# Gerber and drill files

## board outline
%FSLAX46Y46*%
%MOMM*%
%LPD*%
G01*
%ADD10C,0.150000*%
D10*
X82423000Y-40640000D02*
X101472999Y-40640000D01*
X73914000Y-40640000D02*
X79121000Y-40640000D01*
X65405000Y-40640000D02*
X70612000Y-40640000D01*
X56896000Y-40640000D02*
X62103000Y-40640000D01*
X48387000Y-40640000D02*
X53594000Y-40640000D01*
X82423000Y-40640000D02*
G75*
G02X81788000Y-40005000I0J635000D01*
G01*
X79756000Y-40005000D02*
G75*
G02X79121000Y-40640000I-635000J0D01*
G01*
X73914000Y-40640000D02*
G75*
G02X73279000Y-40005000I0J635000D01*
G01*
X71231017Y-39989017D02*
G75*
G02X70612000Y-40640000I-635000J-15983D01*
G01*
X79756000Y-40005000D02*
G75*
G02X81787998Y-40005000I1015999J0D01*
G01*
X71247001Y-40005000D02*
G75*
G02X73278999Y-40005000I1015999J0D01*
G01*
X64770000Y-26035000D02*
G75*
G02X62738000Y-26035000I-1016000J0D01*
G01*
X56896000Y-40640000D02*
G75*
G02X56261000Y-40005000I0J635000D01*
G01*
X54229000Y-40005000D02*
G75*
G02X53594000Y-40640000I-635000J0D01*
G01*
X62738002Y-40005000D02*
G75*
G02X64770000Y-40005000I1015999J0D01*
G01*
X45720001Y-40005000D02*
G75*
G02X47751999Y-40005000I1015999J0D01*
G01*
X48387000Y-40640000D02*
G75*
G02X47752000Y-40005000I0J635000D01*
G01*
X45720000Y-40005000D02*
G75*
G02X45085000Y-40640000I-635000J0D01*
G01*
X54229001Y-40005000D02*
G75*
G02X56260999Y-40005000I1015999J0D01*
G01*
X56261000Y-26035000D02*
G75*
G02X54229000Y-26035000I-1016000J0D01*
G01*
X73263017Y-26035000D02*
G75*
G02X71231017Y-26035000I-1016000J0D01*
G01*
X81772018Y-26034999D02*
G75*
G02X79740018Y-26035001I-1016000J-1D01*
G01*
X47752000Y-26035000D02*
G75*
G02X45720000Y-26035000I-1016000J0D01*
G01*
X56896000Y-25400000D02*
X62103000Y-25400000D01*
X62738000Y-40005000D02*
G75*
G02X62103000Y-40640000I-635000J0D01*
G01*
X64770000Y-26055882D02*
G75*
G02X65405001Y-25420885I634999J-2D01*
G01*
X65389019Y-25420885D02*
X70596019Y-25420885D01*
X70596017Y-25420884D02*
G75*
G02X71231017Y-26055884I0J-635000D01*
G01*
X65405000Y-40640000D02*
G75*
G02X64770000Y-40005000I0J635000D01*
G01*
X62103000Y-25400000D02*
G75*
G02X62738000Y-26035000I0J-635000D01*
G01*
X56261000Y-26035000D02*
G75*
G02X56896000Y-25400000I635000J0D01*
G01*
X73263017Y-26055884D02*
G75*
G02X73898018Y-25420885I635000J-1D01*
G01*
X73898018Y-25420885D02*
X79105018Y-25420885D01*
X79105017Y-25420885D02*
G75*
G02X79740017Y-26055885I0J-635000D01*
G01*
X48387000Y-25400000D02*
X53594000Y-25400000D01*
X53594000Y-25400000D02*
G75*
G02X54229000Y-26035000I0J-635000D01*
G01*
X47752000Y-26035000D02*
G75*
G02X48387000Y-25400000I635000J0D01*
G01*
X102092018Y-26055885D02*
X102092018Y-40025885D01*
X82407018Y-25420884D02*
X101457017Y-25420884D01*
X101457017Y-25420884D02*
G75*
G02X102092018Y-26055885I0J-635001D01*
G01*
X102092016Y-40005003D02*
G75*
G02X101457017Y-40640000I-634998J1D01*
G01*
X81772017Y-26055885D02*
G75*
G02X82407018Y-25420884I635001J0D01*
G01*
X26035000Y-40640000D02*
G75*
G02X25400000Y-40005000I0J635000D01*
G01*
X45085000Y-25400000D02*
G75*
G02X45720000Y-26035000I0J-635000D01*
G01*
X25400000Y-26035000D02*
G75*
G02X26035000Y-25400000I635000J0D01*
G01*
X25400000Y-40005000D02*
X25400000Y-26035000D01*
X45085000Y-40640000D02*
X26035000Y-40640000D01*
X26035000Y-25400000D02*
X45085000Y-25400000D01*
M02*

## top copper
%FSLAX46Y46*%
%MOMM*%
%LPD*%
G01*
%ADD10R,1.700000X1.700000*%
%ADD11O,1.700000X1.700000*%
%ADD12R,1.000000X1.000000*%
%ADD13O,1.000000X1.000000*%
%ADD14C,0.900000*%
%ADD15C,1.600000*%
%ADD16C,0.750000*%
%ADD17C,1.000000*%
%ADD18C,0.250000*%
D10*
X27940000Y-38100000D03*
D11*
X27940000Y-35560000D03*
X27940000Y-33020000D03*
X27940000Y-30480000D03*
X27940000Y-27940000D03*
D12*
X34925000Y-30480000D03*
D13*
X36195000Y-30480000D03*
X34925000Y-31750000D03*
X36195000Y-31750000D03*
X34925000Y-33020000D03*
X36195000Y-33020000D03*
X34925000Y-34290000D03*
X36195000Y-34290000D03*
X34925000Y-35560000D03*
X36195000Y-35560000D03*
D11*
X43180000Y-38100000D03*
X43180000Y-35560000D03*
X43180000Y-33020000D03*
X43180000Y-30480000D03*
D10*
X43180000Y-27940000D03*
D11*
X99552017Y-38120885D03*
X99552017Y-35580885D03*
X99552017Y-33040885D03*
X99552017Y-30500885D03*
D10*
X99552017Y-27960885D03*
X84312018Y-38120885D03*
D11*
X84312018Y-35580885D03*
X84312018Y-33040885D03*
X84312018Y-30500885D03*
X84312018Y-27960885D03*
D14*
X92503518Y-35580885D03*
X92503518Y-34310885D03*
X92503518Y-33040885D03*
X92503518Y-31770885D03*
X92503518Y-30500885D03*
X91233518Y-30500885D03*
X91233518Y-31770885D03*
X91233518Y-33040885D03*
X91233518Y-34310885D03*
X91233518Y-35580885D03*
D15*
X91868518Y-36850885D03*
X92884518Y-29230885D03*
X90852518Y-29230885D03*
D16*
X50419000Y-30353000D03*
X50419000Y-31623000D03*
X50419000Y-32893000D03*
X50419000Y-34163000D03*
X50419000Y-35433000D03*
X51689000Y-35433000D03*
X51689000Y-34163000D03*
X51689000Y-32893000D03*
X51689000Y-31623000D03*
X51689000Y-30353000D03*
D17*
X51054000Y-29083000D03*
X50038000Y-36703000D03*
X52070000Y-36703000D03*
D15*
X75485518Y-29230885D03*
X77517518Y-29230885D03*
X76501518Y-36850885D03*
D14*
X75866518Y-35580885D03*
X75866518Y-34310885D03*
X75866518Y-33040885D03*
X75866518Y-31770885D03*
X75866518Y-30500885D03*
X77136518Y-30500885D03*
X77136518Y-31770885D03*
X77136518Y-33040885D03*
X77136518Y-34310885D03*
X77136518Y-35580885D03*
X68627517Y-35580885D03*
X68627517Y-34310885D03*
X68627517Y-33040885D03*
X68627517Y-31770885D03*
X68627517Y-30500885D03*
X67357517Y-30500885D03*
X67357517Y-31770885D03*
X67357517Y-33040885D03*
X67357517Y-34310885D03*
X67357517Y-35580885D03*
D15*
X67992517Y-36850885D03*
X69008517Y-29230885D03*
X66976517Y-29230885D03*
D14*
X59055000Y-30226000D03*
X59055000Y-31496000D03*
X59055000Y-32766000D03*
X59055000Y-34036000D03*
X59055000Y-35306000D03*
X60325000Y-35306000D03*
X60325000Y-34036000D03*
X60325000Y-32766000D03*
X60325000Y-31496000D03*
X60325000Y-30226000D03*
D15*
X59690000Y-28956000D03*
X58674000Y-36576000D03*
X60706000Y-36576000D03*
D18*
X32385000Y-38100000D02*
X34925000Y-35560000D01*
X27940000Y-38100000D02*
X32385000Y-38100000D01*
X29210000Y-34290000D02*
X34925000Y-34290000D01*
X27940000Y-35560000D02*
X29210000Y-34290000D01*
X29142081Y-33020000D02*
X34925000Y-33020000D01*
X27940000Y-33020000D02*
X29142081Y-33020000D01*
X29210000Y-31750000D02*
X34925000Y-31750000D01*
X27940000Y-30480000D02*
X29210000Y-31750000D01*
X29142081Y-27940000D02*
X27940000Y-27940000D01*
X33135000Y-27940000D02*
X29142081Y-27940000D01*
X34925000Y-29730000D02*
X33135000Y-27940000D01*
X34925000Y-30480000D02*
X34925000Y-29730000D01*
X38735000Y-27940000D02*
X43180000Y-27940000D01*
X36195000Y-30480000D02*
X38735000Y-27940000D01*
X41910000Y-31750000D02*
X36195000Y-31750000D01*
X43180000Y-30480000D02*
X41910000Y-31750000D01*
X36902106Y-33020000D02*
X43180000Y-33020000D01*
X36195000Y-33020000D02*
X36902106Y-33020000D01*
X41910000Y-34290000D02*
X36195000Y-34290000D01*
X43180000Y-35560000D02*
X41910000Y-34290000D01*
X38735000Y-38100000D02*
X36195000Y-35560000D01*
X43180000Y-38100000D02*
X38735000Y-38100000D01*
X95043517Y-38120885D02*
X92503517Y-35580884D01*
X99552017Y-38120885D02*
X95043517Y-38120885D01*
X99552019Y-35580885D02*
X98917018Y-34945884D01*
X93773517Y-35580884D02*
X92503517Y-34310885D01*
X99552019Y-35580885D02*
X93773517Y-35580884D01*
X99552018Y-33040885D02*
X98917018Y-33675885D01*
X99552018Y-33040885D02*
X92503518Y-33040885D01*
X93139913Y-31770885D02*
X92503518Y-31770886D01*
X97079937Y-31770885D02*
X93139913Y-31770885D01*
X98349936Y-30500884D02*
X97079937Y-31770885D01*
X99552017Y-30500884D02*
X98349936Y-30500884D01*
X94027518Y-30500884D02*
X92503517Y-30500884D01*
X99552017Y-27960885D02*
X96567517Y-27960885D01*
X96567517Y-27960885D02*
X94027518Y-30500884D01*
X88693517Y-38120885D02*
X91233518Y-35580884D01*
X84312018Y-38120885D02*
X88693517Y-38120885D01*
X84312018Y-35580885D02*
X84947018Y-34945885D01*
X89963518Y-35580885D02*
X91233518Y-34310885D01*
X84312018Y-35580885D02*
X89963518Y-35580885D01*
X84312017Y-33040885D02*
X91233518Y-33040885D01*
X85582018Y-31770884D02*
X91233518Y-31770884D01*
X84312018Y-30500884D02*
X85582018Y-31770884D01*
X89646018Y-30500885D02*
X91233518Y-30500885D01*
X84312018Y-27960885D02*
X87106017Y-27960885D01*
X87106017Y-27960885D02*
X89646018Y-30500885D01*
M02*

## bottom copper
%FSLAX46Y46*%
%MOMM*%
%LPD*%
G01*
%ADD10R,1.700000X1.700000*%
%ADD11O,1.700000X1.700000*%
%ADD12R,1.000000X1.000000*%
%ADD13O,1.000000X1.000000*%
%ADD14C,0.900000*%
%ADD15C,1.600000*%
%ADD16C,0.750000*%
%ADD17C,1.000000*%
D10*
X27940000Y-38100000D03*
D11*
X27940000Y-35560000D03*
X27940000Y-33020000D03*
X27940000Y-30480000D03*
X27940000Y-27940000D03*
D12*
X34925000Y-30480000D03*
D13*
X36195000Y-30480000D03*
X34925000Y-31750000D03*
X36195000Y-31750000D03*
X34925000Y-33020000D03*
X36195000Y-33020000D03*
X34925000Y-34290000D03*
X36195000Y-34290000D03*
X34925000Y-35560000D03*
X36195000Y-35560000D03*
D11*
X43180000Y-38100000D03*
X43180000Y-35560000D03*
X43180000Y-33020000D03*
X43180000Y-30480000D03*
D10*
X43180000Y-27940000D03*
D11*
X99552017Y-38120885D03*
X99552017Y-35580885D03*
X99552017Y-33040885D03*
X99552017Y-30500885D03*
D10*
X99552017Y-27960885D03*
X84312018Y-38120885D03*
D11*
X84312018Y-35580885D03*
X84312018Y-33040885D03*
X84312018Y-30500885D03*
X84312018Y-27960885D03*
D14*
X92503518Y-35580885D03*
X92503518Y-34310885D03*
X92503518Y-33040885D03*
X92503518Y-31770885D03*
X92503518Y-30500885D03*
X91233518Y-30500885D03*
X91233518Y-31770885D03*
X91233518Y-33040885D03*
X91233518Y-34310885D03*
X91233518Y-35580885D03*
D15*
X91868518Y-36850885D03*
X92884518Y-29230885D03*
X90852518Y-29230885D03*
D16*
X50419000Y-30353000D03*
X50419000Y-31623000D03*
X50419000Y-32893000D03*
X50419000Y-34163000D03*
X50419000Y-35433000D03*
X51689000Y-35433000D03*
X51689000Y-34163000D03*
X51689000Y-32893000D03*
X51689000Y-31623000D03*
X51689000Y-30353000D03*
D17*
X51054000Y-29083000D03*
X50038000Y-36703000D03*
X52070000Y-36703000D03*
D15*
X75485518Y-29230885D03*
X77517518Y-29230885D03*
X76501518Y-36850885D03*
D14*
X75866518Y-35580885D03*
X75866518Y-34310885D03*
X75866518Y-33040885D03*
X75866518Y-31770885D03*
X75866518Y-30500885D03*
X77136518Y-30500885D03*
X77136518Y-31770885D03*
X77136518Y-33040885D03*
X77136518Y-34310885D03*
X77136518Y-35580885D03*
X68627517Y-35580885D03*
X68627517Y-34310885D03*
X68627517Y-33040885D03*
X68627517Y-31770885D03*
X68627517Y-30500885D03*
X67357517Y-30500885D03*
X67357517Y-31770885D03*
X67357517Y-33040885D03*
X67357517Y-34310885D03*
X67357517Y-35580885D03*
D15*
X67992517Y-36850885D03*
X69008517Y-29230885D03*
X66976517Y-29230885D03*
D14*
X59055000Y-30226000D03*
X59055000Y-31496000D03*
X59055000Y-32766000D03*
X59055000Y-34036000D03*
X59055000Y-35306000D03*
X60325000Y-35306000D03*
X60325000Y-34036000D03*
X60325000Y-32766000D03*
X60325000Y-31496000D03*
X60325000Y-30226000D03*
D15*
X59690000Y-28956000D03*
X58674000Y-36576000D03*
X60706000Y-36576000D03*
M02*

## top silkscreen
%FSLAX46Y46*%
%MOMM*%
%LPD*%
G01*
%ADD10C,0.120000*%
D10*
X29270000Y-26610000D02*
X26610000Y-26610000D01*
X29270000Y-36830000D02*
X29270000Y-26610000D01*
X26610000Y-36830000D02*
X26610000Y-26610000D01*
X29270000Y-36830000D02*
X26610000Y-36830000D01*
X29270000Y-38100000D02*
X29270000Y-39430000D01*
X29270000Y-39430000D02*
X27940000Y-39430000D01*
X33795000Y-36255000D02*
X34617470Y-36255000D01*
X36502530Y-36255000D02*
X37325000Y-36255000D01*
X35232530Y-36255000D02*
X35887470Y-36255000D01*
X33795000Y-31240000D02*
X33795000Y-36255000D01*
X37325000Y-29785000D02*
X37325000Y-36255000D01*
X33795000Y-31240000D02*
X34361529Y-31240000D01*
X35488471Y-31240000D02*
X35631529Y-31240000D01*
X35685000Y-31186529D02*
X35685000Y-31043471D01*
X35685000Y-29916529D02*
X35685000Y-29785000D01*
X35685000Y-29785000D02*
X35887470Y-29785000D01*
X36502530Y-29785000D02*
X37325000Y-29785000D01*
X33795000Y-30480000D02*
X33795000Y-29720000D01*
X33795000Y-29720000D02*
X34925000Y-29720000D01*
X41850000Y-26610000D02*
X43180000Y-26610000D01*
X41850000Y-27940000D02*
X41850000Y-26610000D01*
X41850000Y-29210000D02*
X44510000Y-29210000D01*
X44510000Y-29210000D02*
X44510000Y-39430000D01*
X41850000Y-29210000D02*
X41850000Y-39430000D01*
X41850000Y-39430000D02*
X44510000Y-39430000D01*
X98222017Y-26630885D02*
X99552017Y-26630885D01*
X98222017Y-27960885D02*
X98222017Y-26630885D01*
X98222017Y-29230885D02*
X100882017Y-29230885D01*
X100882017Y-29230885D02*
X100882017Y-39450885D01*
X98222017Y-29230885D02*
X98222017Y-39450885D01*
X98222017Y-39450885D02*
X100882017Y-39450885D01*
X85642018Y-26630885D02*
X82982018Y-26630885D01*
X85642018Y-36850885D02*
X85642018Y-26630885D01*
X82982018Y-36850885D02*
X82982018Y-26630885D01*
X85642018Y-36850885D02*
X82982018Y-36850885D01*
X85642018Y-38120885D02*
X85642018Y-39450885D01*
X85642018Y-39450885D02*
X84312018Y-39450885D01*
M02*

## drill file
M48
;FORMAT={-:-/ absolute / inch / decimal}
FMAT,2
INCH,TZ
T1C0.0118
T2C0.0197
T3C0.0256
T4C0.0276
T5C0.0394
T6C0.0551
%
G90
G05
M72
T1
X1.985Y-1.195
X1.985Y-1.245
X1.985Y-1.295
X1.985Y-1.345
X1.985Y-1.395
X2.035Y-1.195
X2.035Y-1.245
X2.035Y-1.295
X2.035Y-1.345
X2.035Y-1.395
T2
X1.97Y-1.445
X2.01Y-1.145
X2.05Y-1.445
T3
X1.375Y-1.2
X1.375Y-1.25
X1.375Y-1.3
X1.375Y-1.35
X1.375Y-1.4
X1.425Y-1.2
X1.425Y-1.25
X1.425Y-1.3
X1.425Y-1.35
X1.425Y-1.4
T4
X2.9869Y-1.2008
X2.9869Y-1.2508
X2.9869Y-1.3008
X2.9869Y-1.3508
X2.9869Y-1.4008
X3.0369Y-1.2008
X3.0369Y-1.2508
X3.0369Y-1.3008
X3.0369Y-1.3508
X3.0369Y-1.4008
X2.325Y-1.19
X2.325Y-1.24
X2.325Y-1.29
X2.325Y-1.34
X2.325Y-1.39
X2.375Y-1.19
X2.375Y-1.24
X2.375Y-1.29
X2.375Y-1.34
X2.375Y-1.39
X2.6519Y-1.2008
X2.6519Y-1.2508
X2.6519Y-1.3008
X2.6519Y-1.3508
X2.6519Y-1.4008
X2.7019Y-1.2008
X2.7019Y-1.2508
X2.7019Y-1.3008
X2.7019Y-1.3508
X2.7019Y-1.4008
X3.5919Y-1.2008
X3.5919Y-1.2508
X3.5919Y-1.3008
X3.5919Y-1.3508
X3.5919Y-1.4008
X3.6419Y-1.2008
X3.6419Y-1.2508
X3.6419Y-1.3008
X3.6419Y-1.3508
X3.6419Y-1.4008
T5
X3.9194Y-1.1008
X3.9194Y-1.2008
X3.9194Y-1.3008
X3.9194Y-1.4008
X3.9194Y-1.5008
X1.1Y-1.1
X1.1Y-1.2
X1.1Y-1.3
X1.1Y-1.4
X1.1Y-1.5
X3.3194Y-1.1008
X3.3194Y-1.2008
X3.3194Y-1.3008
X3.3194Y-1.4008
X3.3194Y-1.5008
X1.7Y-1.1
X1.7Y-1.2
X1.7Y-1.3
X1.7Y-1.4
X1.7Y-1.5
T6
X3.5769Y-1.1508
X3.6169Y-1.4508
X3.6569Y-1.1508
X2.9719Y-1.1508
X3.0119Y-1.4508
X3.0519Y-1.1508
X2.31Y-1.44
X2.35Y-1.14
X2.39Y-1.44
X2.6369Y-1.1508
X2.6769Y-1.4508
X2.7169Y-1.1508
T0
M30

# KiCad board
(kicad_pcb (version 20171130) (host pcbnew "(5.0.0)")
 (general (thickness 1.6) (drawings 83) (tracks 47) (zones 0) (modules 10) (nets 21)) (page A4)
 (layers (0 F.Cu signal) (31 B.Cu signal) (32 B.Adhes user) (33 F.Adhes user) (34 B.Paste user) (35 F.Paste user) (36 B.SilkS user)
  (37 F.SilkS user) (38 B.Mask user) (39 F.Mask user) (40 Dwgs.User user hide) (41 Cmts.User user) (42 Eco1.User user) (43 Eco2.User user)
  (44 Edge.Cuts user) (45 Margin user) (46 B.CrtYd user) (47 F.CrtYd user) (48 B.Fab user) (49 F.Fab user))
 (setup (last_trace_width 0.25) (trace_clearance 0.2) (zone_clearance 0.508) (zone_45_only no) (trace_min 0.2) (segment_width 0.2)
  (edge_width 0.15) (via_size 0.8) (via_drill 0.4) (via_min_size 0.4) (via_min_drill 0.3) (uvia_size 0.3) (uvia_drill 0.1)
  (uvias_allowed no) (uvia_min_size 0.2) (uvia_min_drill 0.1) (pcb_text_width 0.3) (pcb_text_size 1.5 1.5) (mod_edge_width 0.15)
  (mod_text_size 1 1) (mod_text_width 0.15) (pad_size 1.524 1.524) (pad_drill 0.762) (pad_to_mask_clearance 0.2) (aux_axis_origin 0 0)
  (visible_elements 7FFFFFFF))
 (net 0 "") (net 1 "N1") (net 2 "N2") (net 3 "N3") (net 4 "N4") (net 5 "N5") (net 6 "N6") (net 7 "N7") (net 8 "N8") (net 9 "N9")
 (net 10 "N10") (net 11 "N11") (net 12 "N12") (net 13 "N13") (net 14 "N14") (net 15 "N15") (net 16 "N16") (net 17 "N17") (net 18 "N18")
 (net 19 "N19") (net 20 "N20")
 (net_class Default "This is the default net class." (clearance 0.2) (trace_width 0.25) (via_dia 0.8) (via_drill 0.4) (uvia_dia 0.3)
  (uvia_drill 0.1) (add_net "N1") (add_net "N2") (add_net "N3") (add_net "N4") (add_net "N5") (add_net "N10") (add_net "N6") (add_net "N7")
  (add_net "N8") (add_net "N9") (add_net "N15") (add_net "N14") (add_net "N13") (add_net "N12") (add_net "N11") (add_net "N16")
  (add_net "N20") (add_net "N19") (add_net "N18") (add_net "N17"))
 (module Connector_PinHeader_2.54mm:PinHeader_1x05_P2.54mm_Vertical (layer F.Cu) (at 27.94 38.1 180)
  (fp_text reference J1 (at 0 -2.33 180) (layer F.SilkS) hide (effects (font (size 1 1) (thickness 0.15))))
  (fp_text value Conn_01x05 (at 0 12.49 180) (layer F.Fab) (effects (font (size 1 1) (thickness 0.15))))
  (fp_line (start -1.33 11.49) (end 1.33 11.49) (layer F.SilkS) (width 0.12))
  (fp_line (start -1.33 1.27) (end -1.33 11.49) (layer F.SilkS) (width 0.12))
  (fp_line (start 1.33 1.27) (end 1.33 11.49) (layer F.SilkS) (width 0.12))
  (fp_line (start -1.33 1.27) (end 1.33 1.27) (layer F.SilkS) (width 0.12))
  (fp_line (start -1.33 0) (end -1.33 -1.33) (layer F.SilkS) (width 0.12))
  (fp_line (start -1.33 -1.33) (end 0 -1.33) (layer F.SilkS) (width 0.12))
  (pad 1 thru_hole rect (at 0 0 180) (size 1.7 1.7) (drill 1) (layers *.Cu *.Mask) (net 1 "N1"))
  (pad 2 thru_hole oval (at 0 2.54 180) (size 1.7 1.7) (drill 1) (layers *.Cu *.Mask) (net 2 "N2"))
  (pad 3 thru_hole oval (at 0 5.08 180) (size 1.7 1.7) (drill 1) (layers *.Cu *.Mask) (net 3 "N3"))
  (pad 4 thru_hole oval (at 0 7.62 180) (size 1.7 1.7) (drill 1) (layers *.Cu *.Mask) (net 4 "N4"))
  (pad 5 thru_hole oval (at 0 10.16 180) (size 1.7 1.7) (drill 1) (layers *.Cu *.Mask) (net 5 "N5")))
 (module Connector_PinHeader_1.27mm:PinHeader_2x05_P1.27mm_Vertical (layer F.Cu) (at 34.925 30.48)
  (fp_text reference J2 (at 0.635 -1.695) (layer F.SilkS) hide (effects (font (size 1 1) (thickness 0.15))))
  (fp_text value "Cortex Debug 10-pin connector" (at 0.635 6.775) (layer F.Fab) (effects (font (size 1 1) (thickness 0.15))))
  (fp_line (start -1.13 5.775) (end -0.30753 5.775) (layer F.SilkS) (width 0.12))
  (fp_line (start 1.57753 5.775) (end 2.4 5.775) (layer F.SilkS) (width 0.12))
  (fp_line (start 0.30753 5.775) (end 0.96247 5.775) (layer F.SilkS) (width 0.12))
  (fp_line (start -1.13 0.76) (end -1.13 5.775) (layer F.SilkS) (width 0.12))
  (fp_line (start 2.4 -0.695) (end 2.4 5.775) (layer F.SilkS) (width 0.12))
  (fp_line (start -1.13 0.76) (end -0.563471 0.76) (layer F.SilkS) (width 0.12))
  (fp_line (start 0.563471 0.76) (end 0.706529 0.76) (layer F.SilkS) (width 0.12))
  (fp_line (start 0.76 0.706529) (end 0.76 0.563471) (layer F.SilkS) (width 0.12))
  (fp_line (start 0.76 -0.563471) (end 0.76 -0.695) (layer F.SilkS) (width 0.12))
  (fp_line (start 0.76 -0.695) (end 0.96247 -0.695) (layer F.SilkS) (width 0.12))
  (fp_line (start 1.57753 -0.695) (end 2.4 -0.695) (layer F.SilkS) (width 0.12))
  (fp_line (start -1.13 0) (end -1.13 -0.76) (layer F.SilkS) (width 0.12))
  (fp_line (start -1.13 -0.76) (end 0 -0.76) (layer F.SilkS) (width 0.12))
  (pad 1 thru_hole rect (at 0 0) (size 1 1) (drill 0.65) (layers *.Cu *.Mask) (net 5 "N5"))
  (pad 2 thru_hole oval (at 1.27 0) (size 1 1) (drill 0.65) (layers *.Cu *.Mask) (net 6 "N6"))
  (pad 3 thru_hole oval (at 0 1.27) (size 1 1) (drill 0.65) (layers *.Cu *.Mask) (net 4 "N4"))
  (pad 4 thru_hole oval (at 1.27 1.27) (size 1 1) (drill 0.65) (layers *.Cu *.Mask) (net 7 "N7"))
  (pad 5 thru_hole oval (at 0 2.54) (size 1 1) (drill 0.65) (layers *.Cu *.Mask) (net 3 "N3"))
  (pad 6 thru_hole oval (at 1.27 2.54) (size 1 1) (drill 0.65) (layers *.Cu *.Mask) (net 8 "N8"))
  (pad 7 thru_hole oval (at 0 3.81) (size 1 1) (drill 0.65) (layers *.Cu *.Mask) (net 2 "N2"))
  (pad 8 thru_hole oval (at 1.27 3.81) (size 1 1) (drill 0.65) (layers *.Cu *.Mask) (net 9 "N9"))
  (pad 9 thru_hole oval (at 0 5.08) (size 1 1) (drill 0.65) (layers *.Cu *.Mask) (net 1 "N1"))
  (pad 10 thru_hole oval (at 1.27 5.08) (size 1 1) (drill 0.65) (layers *.Cu *.Mask) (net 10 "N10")))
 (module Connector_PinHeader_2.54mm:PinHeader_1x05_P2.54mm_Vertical (layer F.Cu) (at 43.18 27.94)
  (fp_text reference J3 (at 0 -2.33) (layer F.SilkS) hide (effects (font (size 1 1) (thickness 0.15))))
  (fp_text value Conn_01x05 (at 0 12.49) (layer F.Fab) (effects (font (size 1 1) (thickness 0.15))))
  (fp_line (start -1.33 -1.33) (end 0 -1.33) (layer F.SilkS) (width 0.12))
  (fp_line (start -1.33 0) (end -1.33 -1.33) (layer F.SilkS) (width 0.12))
  (fp_line (start -1.33 1.27) (end 1.33 1.27) (layer F.SilkS) (width 0.12))
  (fp_line (start 1.33 1.27) (end 1.33 11.49) (layer F.SilkS) (width 0.12))
  (fp_line (start -1.33 1.27) (end -1.33 11.49) (layer F.SilkS) (width 0.12))
  (fp_line (start -1.33 11.49) (end 1.33 11.49) (layer F.SilkS) (width 0.12))
  (pad 5 thru_hole oval (at 0 10.16) (size 1.7 1.7) (drill 1) (layers *.Cu *.Mask) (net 10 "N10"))
  (pad 4 thru_hole oval (at 0 7.62) (size 1.7 1.7) (drill 1) (layers *.Cu *.Mask) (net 9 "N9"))
  (pad 3 thru_hole oval (at 0 5.08) (size 1.7 1.7) (drill 1) (layers *.Cu *.Mask) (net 8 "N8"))
  (pad 2 thru_hole oval (at 0 2.54) (size 1.7 1.7) (drill 1) (layers *.Cu *.Mask) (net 7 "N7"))
  (pad 1 thru_hole rect (at 0 0) (size 1.7 1.7) (drill 1) (layers *.Cu *.Mask) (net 6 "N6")))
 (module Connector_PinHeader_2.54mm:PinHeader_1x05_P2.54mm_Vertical (layer F.Cu) (at 99.552017 27.960885)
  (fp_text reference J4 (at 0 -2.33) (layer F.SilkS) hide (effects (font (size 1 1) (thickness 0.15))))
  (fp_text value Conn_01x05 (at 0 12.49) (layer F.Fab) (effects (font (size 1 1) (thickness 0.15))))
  (fp_line (start -1.33 -1.33) (end 0 -1.33) (layer F.SilkS) (width 0.12))
  (fp_line (start -1.33 0) (end -1.33 -1.33) (layer F.SilkS) (width 0.12))
  (fp_line (start -1.33 1.27) (end 1.33 1.27) (layer F.SilkS) (width 0.12))
  (fp_line (start 1.33 1.27) (end 1.33 11.49) (layer F.SilkS) (width 0.12))
  (fp_line (start -1.33 1.27) (end -1.33 11.49) (layer F.SilkS) (width 0.12))
  (fp_line (start -1.33 11.49) (end 1.33 11.49) (layer F.SilkS) (width 0.12))
  (pad 5 thru_hole oval (at 0 10.16) (size 1.7 1.7) (drill 1) (layers *.Cu *.Mask) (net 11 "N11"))
  (pad 4 thru_hole oval (at 0 7.62) (size 1.7 1.7) (drill 1) (layers *.Cu *.Mask) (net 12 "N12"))
  (pad 3 thru_hole oval (at 0 5.08) (size 1.7 1.7) (drill 1) (layers *.Cu *.Mask) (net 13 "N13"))
  (pad 2 thru_hole oval (at 0 2.54) (size 1.7 1.7) (drill 1) (layers *.Cu *.Mask) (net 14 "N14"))
  (pad 1 thru_hole rect (at 0 0) (size 1.7 1.7) (drill 1) (layers *.Cu *.Mask) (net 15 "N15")))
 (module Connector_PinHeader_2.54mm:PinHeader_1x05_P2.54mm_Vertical (layer F.Cu) (at 84.312018 38.120885 180)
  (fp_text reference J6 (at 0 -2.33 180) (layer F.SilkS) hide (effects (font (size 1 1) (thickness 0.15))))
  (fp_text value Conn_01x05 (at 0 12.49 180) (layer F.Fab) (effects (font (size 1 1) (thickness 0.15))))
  (fp_line (start -1.33 11.49) (end 1.33 11.49) (layer F.SilkS) (width 0.12))
  (fp_line (start -1.33 1.27) (end -1.33 11.49) (layer F.SilkS) (width 0.12))
  (fp_line (start 1.33 1.27) (end 1.33 11.49) (layer F.SilkS) (width 0.12))
  (fp_line (start -1.33 1.27) (end 1.33 1.27) (layer F.SilkS) (width 0.12))
  (fp_line (start -1.33 0) (end -1.33 -1.33) (layer F.SilkS) (width 0.12))
  (fp_line (start -1.33 -1.33) (end 0 -1.33) (layer F.SilkS) (width 0.12))
  (pad 1 thru_hole rect (at 0 0 180) (size 1.7 1.7) (drill 1) (layers *.Cu *.Mask) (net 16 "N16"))
  (pad 2 thru_hole oval (at 0 2.54 180) (size 1.7 1.7) (drill 1) (layers *.Cu *.Mask) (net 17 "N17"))
  (pad 3 thru_hole oval (at 0 5.08 180) (size 1.7 1.7) (drill 1) (layers *.Cu *.Mask) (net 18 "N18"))
  (pad 4 thru_hole oval (at 0 7.62 180) (size 1.7 1.7) (drill 1) (layers *.Cu *.Mask) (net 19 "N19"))
  (pad 5 thru_hole oval (at 0 10.16 180) (size 1.7 1.7) (drill 1) (layers *.Cu *.Mask) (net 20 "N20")))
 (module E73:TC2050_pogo (layer F.Cu) (at 91.868518 33.040885 180)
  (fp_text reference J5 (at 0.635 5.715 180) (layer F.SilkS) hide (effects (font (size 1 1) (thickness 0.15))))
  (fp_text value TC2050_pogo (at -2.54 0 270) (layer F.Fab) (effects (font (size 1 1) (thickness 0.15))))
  (pad 1 thru_hole circle (at -0.635 -2.54 180) (size 0.9 0.9) (drill 0.7) (layers *.Cu *.Mask) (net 11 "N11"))
  (pad 2 thru_hole circle (at -0.635 -1.27 180) (size 0.9 0.9) (drill 0.7) (layers *.Cu *.Mask) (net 12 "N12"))
  (pad 3 thru_hole circle (at -0.635 0 180) (size 0.9 0.9) (drill 0.7) (layers *.Cu *.Mask) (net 13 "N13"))
  (pad 4 thru_hole circle (at -0.635 1.27 180) (size 0.9 0.9) (drill 0.7) (layers *.Cu *.Mask) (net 14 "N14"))
  (pad 5 thru_hole circle (at -0.635 2.54 180) (size 0.9 0.9) (drill 0.7) (layers *.Cu *.Mask) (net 15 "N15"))
  (pad 6 thru_hole circle (at 0.635 2.54 180) (size 0.9 0.9) (drill 0.7) (layers *.Cu *.Mask) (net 20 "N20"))
  (pad 7 thru_hole circle (at 0.635 1.27 180) (size 0.9 0.9) (drill 0.7) (layers *.Cu *.Mask) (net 19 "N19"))
  (pad 8 thru_hole circle (at 0.635 0 180) (size 0.9 0.9) (drill 0.7) (layers *.Cu *.Mask) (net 18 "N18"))
  (pad 9 thru_hole circle (at 0.635 -1.27 180) (size 0.9 0.9) (drill 0.7) (layers *.Cu *.Mask) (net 17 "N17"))
  (pad 10 thru_hole circle (at 0.635 -2.54 180) (size 0.9 0.9) (drill 0.7) (layers *.Cu *.Mask) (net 16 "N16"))
  (pad "" thru_hole circle (at 0 -3.81 180) (size 1.6 1.6) (drill 1.4) (layers *.Cu *.Mask))
  (pad "" thru_hole circle (at -1.016 3.81 180) (size 1.6 1.6) (drill 1.4) (layers *.Cu *.Mask))
  (pad "" thru_hole circle (at 1.016 3.81 180) (size 1.6 1.6) (drill 1.4) (layers *.Cu *.Mask)))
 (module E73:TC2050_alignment (layer F.Cu) (at 51.054 32.893)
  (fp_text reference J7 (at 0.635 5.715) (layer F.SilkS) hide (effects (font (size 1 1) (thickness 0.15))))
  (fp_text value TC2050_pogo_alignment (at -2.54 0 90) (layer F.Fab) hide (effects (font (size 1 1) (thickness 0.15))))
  (pad 1 thru_hole circle (at -0.635 -2.54) (size 0.75 0.75) (drill 0.3) (layers *.Cu *.Mask))
  (pad 2 thru_hole circle (at -0.635 -1.27) (size 0.75 0.75) (drill 0.3) (layers *.Cu *.Mask))
  (pad 3 thru_hole circle (at -0.635 0) (size 0.75 0.75) (drill 0.3) (layers *.Cu *.Mask))
  (pad 4 thru_hole circle (at -0.635 1.27) (size 0.75 0.75) (drill 0.3) (layers *.Cu *.Mask))
  (pad 5 thru_hole circle (at -0.635 2.54) (size 0.75 0.75) (drill 0.3) (layers *.Cu *.Mask))
  (pad 6 thru_hole circle (at 0.635 2.54) (size 0.75 0.75) (drill 0.3) (layers *.Cu *.Mask))
  (pad 7 thru_hole circle (at 0.635 1.27) (size 0.75 0.75) (drill 0.3) (layers *.Cu *.Mask))
  (pad 8 thru_hole circle (at 0.635 0) (size 0.75 0.75) (drill 0.3) (layers *.Cu *.Mask))
  (pad 9 thru_hole circle (at 0.635 -1.27) (size 0.75 0.75) (drill 0.3) (layers *.Cu *.Mask))
  (pad 10 thru_hole circle (at 0.635 -2.54) (size 0.75 0.75) (drill 0.3) (layers *.Cu *.Mask))
  (pad "" thru_hole circle (at 0 -3.81) (size 1 1) (drill 0.5) (layers *.Cu *.Mask))
  (pad "" thru_hole circle (at -1.016 3.81) (size 1 1) (drill 0.5) (layers *.Cu *.Mask))
  (pad "" thru_hole circle (at 1.016 3.81) (size 1 1) (drill 0.5) (layers *.Cu *.Mask)))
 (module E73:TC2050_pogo (layer F.Cu) (at 76.501518 33.040885 180)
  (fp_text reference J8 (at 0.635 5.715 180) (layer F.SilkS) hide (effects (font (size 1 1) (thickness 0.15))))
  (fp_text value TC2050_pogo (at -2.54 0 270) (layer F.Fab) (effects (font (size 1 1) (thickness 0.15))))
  (pad "" thru_hole circle (at 1.016 3.81 180) (size 1.6 1.6) (drill 1.4) (layers *.Cu *.Mask))
  (pad "" thru_hole circle (at -1.016 3.81 180) (size 1.6 1.6) (drill 1.4) (layers *.Cu *.Mask))
  (pad "" thru_hole circle (at 0 -3.81 180) (size 1.6 1.6) (drill 1.4) (layers *.Cu *.Mask))
  (pad 10 thru_hole circle (at 0.635 -2.54 180) (size 0.9 0.9) (drill 0.7) (layers *.Cu *.Mask))
  (pad 9 thru_hole circle (at 0.635 -1.27 180) (size 0.9 0.9) (drill 0.7) (layers *.Cu *.Mask))
  (pad 8 thru_hole circle (at 0.635 0 180) (size 0.9 0.9) (drill 0.7) (layers *.Cu *.Mask))
  (pad 7 thru_hole circle (at 0.635 1.27 180) (size 0.9 0.9) (drill 0.7) (layers *.Cu *.Mask))
  (pad 6 thru_hole circle (at 0.635 2.54 180) (size 0.9 0.9) (drill 0.7) (layers *.Cu *.Mask))
  (pad 5 thru_hole circle (at -0.635 2.54 180) (size 0.9 0.9) (drill 0.7) (layers *.Cu *.Mask))
  (pad 4 thru_hole circle (at -0.635 1.27 180) (size 0.9 0.9) (drill 0.7) (layers *.Cu *.Mask))
  (pad 3 thru_hole circle (at -0.635 0 180) (size 0.9 0.9) (drill 0.7) (layers *.Cu *.Mask))
  (pad 2 thru_hole circle (at -0.635 -1.27 180) (size 0.9 0.9) (drill 0.7) (layers *.Cu *.Mask))
  (pad 1 thru_hole circle (at -0.635 -2.54 180) (size 0.9 0.9) (drill 0.7) (layers *.Cu *.Mask)))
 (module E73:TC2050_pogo (layer F.Cu) (at 67.992517 33.040885 180)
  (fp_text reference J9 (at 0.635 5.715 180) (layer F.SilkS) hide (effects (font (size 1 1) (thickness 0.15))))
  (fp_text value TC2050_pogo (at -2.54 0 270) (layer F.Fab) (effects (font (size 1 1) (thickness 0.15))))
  (pad 1 thru_hole circle (at -0.635 -2.54 180) (size 0.9 0.9) (drill 0.7) (layers *.Cu *.Mask))
  (pad 2 thru_hole circle (at -0.635 -1.27 180) (size 0.9 0.9) (drill 0.7) (layers *.Cu *.Mask))
  (pad 3 thru_hole circle (at -0.635 0 180) (size 0.9 0.9) (drill 0.7) (layers *.Cu *.Mask))
  (pad 4 thru_hole circle (at -0.635 1.27 180) (size 0.9 0.9) (drill 0.7) (layers *.Cu *.Mask))
  (pad 5 thru_hole circle (at -0.635 2.54 180) (size 0.9 0.9) (drill 0.7) (layers *.Cu *.Mask))
  (pad 6 thru_hole circle (at 0.635 2.54 180) (size 0.9 0.9) (drill 0.7) (layers *.Cu *.Mask))
  (pad 7 thru_hole circle (at 0.635 1.27 180) (size 0.9 0.9) (drill 0.7) (layers *.Cu *.Mask))
  (pad 8 thru_hole circle (at 0.635 0 180) (size 0.9 0.9) (drill 0.7) (layers *.Cu *.Mask))
  (pad 9 thru_hole circle (at 0.635 -1.27 180) (size 0.9 0.9) (drill 0.7) (layers *.Cu *.Mask))
  (pad 10 thru_hole circle (at 0.635 -2.54 180) (size 0.9 0.9) (drill 0.7) (layers *.Cu *.Mask))
  (pad "" thru_hole circle (at 0 -3.81 180) (size 1.6 1.6) (drill 1.4) (layers *.Cu *.Mask))
  (pad "" thru_hole circle (at -1.016 3.81 180) (size 1.6 1.6) (drill 1.4) (layers *.Cu *.Mask))
  (pad "" thru_hole circle (at 1.016 3.81 180) (size 1.6 1.6) (drill 1.4) (layers *.Cu *.Mask)))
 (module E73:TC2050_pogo (layer F.Cu) (at 59.69 32.766)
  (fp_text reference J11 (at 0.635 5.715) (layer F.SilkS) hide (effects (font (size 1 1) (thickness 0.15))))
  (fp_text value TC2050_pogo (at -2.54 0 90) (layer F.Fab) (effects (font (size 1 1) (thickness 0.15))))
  (pad 1 thru_hole circle (at -0.635 -2.54) (size 0.9 0.9) (drill 0.7) (layers *.Cu *.Mask))
  (pad 2 thru_hole circle (at -0.635 -1.27) (size 0.9 0.9) (drill 0.7) (layers *.Cu *.Mask))
  (pad 3 thru_hole circle (at -0.635 0) (size 0.9 0.9) (drill 0.7) (layers *.Cu *.Mask))
  (pad 4 thru_hole circle (at -0.635 1.27) (size 0.9 0.9) (drill 0.7) (layers *.Cu *.Mask))
  (pad 5 thru_hole circle (at -0.635 2.54) (size 0.9 0.9) (drill 0.7) (layers *.Cu *.Mask))
  (pad 6 thru_hole circle (at 0.635 2.54) (size 0.9 0.9) (drill 0.7) (layers *.Cu *.Mask))
  (pad 7 thru_hole circle (at 0.635 1.27) (size 0.9 0.9) (drill 0.7) (layers *.Cu *.Mask))
  (pad 8 thru_hole circle (at 0.635 0) (size 0.9 0.9) (drill 0.7) (layers *.Cu *.Mask))
  (pad 9 thru_hole circle (at 0.635 -1.27) (size 0.9 0.9) (drill 0.7) (layers *.Cu *.Mask))
  (pad 10 thru_hole circle (at 0.635 -2.54) (size 0.9 0.9) (drill 0.7) (layers *.Cu *.Mask))
  (pad "" thru_hole circle (at 0 -3.81) (size 1.6 1.6) (drill 1.4) (layers *.Cu *.Mask))
  (pad "" thru_hole circle (at -1.016 3.81) (size 1.6 1.6) (drill 1.4) (layers *.Cu *.Mask))
  (pad "" thru_hole circle (at 1.016 3.81) (size 1.6 1.6) (drill 1.4) (layers *.Cu *.Mask)))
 (gr_line (start 82.423 40.64) (end 101.472999 40.64) (layer Edge.Cuts) (width 0.15))
 (gr_line (start 73.914 40.64) (end 79.121 40.64) (layer Edge.Cuts) (width 0.15))
 (gr_line (start 65.405 40.64) (end 70.612 40.64) (layer Edge.Cuts) (width 0.15))
 (gr_line (start 56.896 40.64) (end 62.103 40.64) (layer Edge.Cuts) (width 0.15))
 (gr_line (start 48.387 40.64) (end 53.594 40.64) (layer Edge.Cuts) (width 0.15))
 (gr_arc (start 82.423 40.005) (end 81.788 40.005) (angle -90) (layer Edge.Cuts) (width 0.15))
 (gr_arc (start 79.121 40.005) (end 79.121 40.64) (angle -90) (layer Edge.Cuts) (width 0.15))
 (gr_arc (start 73.914 40.005) (end 73.279 40.005) (angle -90) (layer Edge.Cuts) (width 0.15))
 (gr_arc (start 70.596017 40.005) (end 70.612 40.64) (angle -90) (layer Edge.Cuts) (width 0.15))
 (gr_arc (start 80.771999 40.005) (end 81.787998 40.005) (angle -180) (layer Edge.Cuts) (width 0.15))
 (gr_arc (start 72.263 40.005) (end 73.278999 40.005) (angle -180) (layer Edge.Cuts) (width 0.15))
 (gr_arc (start 63.754 26.035) (end 62.738 26.035) (angle -180) (layer Edge.Cuts) (width 0.15))
 (gr_arc (start 56.896 40.005) (end 56.261 40.005) (angle -90) (layer Edge.Cuts) (width 0.15))
 (gr_arc (start 53.594 40.005) (end 53.594 40.64) (angle -90) (layer Edge.Cuts) (width 0.15))
 (gr_arc (start 63.754001 40.005) (end 64.77 40.005) (angle -180) (layer Edge.Cuts) (width 0.15))
 (gr_arc (start 46.736 40.005) (end 47.751999 40.005) (angle -180) (layer Edge.Cuts) (width 0.15))
 (gr_arc (start 48.387 40.005) (end 47.752 40.005) (angle -90) (layer Edge.Cuts) (width 0.15))
 (gr_arc (start 45.085 40.005) (end 45.085 40.64) (angle -90) (layer Edge.Cuts) (width 0.15))
 (gr_arc (start 55.245 40.005) (end 56.260999 40.005) (angle -180) (layer Edge.Cuts) (width 0.15))
 (gr_arc (start 55.245 26.035) (end 54.229 26.035) (angle -180) (layer Edge.Cuts) (width 0.15))
 (gr_arc (start 72.247017 26.035) (end 71.231017 26.035) (angle -180) (layer Edge.Cuts) (width 0.15))
 (gr_arc (start 80.756018 26.035) (end 79.740018 26.035001) (angle -180) (layer Edge.Cuts) (width 0.15))
 (gr_arc (start 46.736 26.035) (end 45.72 26.035) (angle -180) (layer Edge.Cuts) (width 0.15))
 (gr_line (start 56.896 25.4) (end 62.103 25.4) (layer Edge.Cuts) (width 0.15))
 (gr_arc (start 62.103 40.005) (end 62.103 40.64) (angle -90) (layer Edge.Cuts) (width 0.15))
 (gr_arc (start 65.404999 26.055884) (end 65.405001 25.420885) (angle -90) (layer Edge.Cuts) (width 0.15))
 (gr_line (start 65.389019 25.420885) (end 70.596019 25.420885) (layer Edge.Cuts) (width 0.15))
 (gr_arc (start 70.596017 26.055884) (end 71.231017 26.055884) (angle -90) (layer Edge.Cuts) (width 0.15))
 (gr_arc (start 65.405 40.005) (end 64.77 40.005) (angle -90) (layer Edge.Cuts) (width 0.15))
 (gr_arc (start 62.103 26.035) (end 62.738 26.035) (angle -90) (layer Edge.Cuts) (width 0.15))
 (gr_arc (start 56.896 26.035) (end 56.896 25.4) (angle -90) (layer Edge.Cuts) (width 0.15))
 (gr_arc (start 73.898017 26.055885) (end 73.898018 25.420885) (angle -90) (layer Edge.Cuts) (width 0.15))
 (gr_line (start 73.898018 25.420885) (end 79.105018 25.420885) (layer Edge.Cuts) (width 0.15))
 (gr_arc (start 79.105017 26.055885) (end 79.740017 26.055885) (angle -90) (layer Edge.Cuts) (width 0.15))
 (gr_line (start 48.387 25.4) (end 53.594 25.4) (layer Edge.Cuts) (width 0.15))
 (gr_arc (start 53.594 26.035) (end 54.229 26.035) (angle -90) (layer Edge.Cuts) (width 0.15))
 (gr_arc (start 48.387 26.035) (end 48.387 25.4) (angle -90) (layer Edge.Cuts) (width 0.15))
 (gr_line (start 102.092018 26.055885) (end 102.092018 40.025885) (layer Edge.Cuts) (width 0.15))
 (gr_line (start 82.407018 25.420884) (end 101.457017 25.420884) (layer Edge.Cuts) (width 0.15))
 (gr_arc (start 101.457017 26.055885) (end 102.092018 26.055885) (angle -90) (layer Edge.Cuts) (width 0.15))
 (gr_arc (start 101.457018 40.005002) (end 101.457017 40.64) (angle -90) (layer Edge.Cuts) (width 0.15))
 (gr_arc (start 82.407018 26.055885) (end 82.407018 25.420884) (angle -90) (layer Edge.Cuts) (width 0.15))
 (gr_arc (start 26.035 40.005) (end 25.4 40.005) (angle -90) (layer Edge.Cuts) (width 0.15))
 (gr_arc (start 45.085 26.035) (end 45.72 26.035) (angle -90) (layer Edge.Cuts) (width 0.15))
 (gr_arc (start 26.035 26.035) (end 26.035 25.4) (angle -90) (layer Edge.Cuts) (width 0.15))
 (gr_line (start 25.4 40.005) (end 25.4 26.035) (layer Edge.Cuts) (width 0.15))
 (gr_line (start 45.085 40.64) (end 26.035 40.64) (layer Edge.Cuts) (width 0.15))
 (gr_line (start 26.035 25.4) (end 45.085 25.4) (layer Edge.Cuts) (width 0.15))
 (segment (start 32.385 38.1) (end 34.925 35.56) (width 0.25) (layer F.Cu) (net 1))
 (segment (start 27.94 38.1) (end 32.385 38.1) (width 0.25) (layer F.Cu) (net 1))
 (segment (start 29.21 34.29) (end 34.925 34.29) (width 0.25) (layer F.Cu) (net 2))
 (segment (start 27.94 35.56) (end 29.21 34.29) (width 0.25) (layer F.Cu) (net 2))
 (segment (start 29.142081 33.02) (end 34.925 33.02) (width 0.25) (layer F.Cu) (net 3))
 (segment (start 27.94 33.02) (end 29.142081 33.02) (width 0.25) (layer F.Cu) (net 3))
 (segment (start 29.21 31.75) (end 34.925 31.75) (width 0.25) (layer F.Cu) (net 4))
 (segment (start 27.94 30.48) (end 29.21 31.75) (width 0.25) (layer F.Cu) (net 4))
 (segment (start 29.142081 27.94) (end 27.94 27.94) (width 0.25) (layer F.Cu) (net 5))
 (segment (start 33.135 27.94) (end 29.142081 27.94) (width 0.25) (layer F.Cu) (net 5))
 (segment (start 34.925 29.73) (end 33.135 27.94) (width 0.25) (layer F.Cu) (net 5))
 (segment (start 34.925 30.48) (end 34.925 29.73) (width 0.25) (layer F.Cu) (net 5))
 (segment (start 38.735 27.94) (end 43.18 27.94) (width 0.25) (layer F.Cu) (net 6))
 (segment (start 36.195 30.48) (end 38.735 27.94) (width 0.25) (layer F.Cu) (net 6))
 (segment (start 41.91 31.75) (end 36.195 31.75) (width 0.25) (layer F.Cu) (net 7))
 (segment (start 43.18 30.48) (end 41.91 31.75) (width 0.25) (layer F.Cu) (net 7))
 (segment (start 36.902106 33.02) (end 43.18 33.02) (width 0.25) (layer F.Cu) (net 8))
 (segment (start 36.195 33.02) (end 36.902106 33.02) (width 0.25) (layer F.Cu) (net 8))
 (segment (start 41.91 34.29) (end 36.195 34.29) (width 0.25) (layer F.Cu) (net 9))
 (segment (start 43.18 35.56) (end 41.91 34.29) (width 0.25) (layer F.Cu) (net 9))
 (segment (start 38.735 38.1) (end 36.195 35.56) (width 0.25) (layer F.Cu) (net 10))
 (segment (start 43.18 38.1) (end 38.735 38.1) (width 0.25) (layer F.Cu) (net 10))
 (segment (start 95.043517 38.120885) (end 92.503517 35.580884) (width 0.25) (layer F.Cu) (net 11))
 (segment (start 99.552017 38.120885) (end 95.043517 38.120885) (width 0.25) (layer F.Cu) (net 11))
 (segment (start 99.552019 35.580885) (end 98.917018 34.945884) (width 0.25) (layer F.Cu) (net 12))
 (segment (start 93.773517 35.580884) (end 92.503517 34.310885) (width 0.25) (layer F.Cu) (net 12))
 (segment (start 99.552019 35.580885) (end 93.773517 35.580884) (width 0.25) (layer F.Cu) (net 12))
 (segment (start 99.552018 33.040885) (end 98.917018 33.675885) (width 0.25) (layer F.Cu) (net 13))
 (segment (start 99.552018 33.040885) (end 92.503518 33.040885) (width 0.25) (layer F.Cu) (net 13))
 (segment (start 93.139913 31.770885) (end 92.503518 31.770886) (width 0.25) (layer F.Cu) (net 14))
 (segment (start 97.079937 31.770885) (end 93.139913 31.770885) (width 0.25) (layer F.Cu) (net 14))
 (segment (start 98.349936 30.500884) (end 97.079937 31.770885) (width 0.25) (layer F.Cu) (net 14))
 (segment (start 99.552017 30.500884) (end 98.349936 30.500884) (width 0.25) (layer F.Cu) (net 14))
 (segment (start 94.027518 30.500884) (end 92.503517 30.500884) (width 0.25) (layer F.Cu) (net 15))
 (segment (start 99.552017 27.960885) (end 96.567517 27.960885) (width 0.25) (layer F.Cu) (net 15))
 (segment (start 96.567517 27.960885) (end 94.027518 30.500884) (width 0.25) (layer F.Cu) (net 15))
 (segment (start 88.693517 38.120885) (end 91.233518 35.580884) (width 0.25) (layer F.Cu) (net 16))
 (segment (start 84.312018 38.120885) (end 88.693517 38.120885) (width 0.25) (layer F.Cu) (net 16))
 (segment (start 84.312018 35.580885) (end 84.947018 34.945885) (width 0.25) (layer F.Cu) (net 17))
 (segment (start 89.963518 35.580885) (end 91.233518 34.310885) (width 0.25) (layer F.Cu) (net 17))
 (segment (start 84.312018 35.580885) (end 89.963518 35.580885) (width 0.25) (layer F.Cu) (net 17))
 (segment (start 84.312017 33.040885) (end 91.233518 33.040885) (width 0.25) (layer F.Cu) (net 18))
 (segment (start 85.582018 31.770884) (end 91.233518 31.770884) (width 0.25) (layer F.Cu) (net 19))
 (segment (start 84.312018 30.500884) (end 85.582018 31.770884) (width 0.25) (layer F.Cu) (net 19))
 (segment (start 89.646018 30.500885) (end 91.233518 30.500885) (width 0.25) (layer F.Cu) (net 20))
 (segment (start 84.312018 27.960885) (end 87.106017 27.960885) (width 0.25) (layer F.Cu) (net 20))
 (segment (start 87.106017 27.960885) (end 89.646018 30.500885) (width 0.25) (layer F.Cu) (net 20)))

